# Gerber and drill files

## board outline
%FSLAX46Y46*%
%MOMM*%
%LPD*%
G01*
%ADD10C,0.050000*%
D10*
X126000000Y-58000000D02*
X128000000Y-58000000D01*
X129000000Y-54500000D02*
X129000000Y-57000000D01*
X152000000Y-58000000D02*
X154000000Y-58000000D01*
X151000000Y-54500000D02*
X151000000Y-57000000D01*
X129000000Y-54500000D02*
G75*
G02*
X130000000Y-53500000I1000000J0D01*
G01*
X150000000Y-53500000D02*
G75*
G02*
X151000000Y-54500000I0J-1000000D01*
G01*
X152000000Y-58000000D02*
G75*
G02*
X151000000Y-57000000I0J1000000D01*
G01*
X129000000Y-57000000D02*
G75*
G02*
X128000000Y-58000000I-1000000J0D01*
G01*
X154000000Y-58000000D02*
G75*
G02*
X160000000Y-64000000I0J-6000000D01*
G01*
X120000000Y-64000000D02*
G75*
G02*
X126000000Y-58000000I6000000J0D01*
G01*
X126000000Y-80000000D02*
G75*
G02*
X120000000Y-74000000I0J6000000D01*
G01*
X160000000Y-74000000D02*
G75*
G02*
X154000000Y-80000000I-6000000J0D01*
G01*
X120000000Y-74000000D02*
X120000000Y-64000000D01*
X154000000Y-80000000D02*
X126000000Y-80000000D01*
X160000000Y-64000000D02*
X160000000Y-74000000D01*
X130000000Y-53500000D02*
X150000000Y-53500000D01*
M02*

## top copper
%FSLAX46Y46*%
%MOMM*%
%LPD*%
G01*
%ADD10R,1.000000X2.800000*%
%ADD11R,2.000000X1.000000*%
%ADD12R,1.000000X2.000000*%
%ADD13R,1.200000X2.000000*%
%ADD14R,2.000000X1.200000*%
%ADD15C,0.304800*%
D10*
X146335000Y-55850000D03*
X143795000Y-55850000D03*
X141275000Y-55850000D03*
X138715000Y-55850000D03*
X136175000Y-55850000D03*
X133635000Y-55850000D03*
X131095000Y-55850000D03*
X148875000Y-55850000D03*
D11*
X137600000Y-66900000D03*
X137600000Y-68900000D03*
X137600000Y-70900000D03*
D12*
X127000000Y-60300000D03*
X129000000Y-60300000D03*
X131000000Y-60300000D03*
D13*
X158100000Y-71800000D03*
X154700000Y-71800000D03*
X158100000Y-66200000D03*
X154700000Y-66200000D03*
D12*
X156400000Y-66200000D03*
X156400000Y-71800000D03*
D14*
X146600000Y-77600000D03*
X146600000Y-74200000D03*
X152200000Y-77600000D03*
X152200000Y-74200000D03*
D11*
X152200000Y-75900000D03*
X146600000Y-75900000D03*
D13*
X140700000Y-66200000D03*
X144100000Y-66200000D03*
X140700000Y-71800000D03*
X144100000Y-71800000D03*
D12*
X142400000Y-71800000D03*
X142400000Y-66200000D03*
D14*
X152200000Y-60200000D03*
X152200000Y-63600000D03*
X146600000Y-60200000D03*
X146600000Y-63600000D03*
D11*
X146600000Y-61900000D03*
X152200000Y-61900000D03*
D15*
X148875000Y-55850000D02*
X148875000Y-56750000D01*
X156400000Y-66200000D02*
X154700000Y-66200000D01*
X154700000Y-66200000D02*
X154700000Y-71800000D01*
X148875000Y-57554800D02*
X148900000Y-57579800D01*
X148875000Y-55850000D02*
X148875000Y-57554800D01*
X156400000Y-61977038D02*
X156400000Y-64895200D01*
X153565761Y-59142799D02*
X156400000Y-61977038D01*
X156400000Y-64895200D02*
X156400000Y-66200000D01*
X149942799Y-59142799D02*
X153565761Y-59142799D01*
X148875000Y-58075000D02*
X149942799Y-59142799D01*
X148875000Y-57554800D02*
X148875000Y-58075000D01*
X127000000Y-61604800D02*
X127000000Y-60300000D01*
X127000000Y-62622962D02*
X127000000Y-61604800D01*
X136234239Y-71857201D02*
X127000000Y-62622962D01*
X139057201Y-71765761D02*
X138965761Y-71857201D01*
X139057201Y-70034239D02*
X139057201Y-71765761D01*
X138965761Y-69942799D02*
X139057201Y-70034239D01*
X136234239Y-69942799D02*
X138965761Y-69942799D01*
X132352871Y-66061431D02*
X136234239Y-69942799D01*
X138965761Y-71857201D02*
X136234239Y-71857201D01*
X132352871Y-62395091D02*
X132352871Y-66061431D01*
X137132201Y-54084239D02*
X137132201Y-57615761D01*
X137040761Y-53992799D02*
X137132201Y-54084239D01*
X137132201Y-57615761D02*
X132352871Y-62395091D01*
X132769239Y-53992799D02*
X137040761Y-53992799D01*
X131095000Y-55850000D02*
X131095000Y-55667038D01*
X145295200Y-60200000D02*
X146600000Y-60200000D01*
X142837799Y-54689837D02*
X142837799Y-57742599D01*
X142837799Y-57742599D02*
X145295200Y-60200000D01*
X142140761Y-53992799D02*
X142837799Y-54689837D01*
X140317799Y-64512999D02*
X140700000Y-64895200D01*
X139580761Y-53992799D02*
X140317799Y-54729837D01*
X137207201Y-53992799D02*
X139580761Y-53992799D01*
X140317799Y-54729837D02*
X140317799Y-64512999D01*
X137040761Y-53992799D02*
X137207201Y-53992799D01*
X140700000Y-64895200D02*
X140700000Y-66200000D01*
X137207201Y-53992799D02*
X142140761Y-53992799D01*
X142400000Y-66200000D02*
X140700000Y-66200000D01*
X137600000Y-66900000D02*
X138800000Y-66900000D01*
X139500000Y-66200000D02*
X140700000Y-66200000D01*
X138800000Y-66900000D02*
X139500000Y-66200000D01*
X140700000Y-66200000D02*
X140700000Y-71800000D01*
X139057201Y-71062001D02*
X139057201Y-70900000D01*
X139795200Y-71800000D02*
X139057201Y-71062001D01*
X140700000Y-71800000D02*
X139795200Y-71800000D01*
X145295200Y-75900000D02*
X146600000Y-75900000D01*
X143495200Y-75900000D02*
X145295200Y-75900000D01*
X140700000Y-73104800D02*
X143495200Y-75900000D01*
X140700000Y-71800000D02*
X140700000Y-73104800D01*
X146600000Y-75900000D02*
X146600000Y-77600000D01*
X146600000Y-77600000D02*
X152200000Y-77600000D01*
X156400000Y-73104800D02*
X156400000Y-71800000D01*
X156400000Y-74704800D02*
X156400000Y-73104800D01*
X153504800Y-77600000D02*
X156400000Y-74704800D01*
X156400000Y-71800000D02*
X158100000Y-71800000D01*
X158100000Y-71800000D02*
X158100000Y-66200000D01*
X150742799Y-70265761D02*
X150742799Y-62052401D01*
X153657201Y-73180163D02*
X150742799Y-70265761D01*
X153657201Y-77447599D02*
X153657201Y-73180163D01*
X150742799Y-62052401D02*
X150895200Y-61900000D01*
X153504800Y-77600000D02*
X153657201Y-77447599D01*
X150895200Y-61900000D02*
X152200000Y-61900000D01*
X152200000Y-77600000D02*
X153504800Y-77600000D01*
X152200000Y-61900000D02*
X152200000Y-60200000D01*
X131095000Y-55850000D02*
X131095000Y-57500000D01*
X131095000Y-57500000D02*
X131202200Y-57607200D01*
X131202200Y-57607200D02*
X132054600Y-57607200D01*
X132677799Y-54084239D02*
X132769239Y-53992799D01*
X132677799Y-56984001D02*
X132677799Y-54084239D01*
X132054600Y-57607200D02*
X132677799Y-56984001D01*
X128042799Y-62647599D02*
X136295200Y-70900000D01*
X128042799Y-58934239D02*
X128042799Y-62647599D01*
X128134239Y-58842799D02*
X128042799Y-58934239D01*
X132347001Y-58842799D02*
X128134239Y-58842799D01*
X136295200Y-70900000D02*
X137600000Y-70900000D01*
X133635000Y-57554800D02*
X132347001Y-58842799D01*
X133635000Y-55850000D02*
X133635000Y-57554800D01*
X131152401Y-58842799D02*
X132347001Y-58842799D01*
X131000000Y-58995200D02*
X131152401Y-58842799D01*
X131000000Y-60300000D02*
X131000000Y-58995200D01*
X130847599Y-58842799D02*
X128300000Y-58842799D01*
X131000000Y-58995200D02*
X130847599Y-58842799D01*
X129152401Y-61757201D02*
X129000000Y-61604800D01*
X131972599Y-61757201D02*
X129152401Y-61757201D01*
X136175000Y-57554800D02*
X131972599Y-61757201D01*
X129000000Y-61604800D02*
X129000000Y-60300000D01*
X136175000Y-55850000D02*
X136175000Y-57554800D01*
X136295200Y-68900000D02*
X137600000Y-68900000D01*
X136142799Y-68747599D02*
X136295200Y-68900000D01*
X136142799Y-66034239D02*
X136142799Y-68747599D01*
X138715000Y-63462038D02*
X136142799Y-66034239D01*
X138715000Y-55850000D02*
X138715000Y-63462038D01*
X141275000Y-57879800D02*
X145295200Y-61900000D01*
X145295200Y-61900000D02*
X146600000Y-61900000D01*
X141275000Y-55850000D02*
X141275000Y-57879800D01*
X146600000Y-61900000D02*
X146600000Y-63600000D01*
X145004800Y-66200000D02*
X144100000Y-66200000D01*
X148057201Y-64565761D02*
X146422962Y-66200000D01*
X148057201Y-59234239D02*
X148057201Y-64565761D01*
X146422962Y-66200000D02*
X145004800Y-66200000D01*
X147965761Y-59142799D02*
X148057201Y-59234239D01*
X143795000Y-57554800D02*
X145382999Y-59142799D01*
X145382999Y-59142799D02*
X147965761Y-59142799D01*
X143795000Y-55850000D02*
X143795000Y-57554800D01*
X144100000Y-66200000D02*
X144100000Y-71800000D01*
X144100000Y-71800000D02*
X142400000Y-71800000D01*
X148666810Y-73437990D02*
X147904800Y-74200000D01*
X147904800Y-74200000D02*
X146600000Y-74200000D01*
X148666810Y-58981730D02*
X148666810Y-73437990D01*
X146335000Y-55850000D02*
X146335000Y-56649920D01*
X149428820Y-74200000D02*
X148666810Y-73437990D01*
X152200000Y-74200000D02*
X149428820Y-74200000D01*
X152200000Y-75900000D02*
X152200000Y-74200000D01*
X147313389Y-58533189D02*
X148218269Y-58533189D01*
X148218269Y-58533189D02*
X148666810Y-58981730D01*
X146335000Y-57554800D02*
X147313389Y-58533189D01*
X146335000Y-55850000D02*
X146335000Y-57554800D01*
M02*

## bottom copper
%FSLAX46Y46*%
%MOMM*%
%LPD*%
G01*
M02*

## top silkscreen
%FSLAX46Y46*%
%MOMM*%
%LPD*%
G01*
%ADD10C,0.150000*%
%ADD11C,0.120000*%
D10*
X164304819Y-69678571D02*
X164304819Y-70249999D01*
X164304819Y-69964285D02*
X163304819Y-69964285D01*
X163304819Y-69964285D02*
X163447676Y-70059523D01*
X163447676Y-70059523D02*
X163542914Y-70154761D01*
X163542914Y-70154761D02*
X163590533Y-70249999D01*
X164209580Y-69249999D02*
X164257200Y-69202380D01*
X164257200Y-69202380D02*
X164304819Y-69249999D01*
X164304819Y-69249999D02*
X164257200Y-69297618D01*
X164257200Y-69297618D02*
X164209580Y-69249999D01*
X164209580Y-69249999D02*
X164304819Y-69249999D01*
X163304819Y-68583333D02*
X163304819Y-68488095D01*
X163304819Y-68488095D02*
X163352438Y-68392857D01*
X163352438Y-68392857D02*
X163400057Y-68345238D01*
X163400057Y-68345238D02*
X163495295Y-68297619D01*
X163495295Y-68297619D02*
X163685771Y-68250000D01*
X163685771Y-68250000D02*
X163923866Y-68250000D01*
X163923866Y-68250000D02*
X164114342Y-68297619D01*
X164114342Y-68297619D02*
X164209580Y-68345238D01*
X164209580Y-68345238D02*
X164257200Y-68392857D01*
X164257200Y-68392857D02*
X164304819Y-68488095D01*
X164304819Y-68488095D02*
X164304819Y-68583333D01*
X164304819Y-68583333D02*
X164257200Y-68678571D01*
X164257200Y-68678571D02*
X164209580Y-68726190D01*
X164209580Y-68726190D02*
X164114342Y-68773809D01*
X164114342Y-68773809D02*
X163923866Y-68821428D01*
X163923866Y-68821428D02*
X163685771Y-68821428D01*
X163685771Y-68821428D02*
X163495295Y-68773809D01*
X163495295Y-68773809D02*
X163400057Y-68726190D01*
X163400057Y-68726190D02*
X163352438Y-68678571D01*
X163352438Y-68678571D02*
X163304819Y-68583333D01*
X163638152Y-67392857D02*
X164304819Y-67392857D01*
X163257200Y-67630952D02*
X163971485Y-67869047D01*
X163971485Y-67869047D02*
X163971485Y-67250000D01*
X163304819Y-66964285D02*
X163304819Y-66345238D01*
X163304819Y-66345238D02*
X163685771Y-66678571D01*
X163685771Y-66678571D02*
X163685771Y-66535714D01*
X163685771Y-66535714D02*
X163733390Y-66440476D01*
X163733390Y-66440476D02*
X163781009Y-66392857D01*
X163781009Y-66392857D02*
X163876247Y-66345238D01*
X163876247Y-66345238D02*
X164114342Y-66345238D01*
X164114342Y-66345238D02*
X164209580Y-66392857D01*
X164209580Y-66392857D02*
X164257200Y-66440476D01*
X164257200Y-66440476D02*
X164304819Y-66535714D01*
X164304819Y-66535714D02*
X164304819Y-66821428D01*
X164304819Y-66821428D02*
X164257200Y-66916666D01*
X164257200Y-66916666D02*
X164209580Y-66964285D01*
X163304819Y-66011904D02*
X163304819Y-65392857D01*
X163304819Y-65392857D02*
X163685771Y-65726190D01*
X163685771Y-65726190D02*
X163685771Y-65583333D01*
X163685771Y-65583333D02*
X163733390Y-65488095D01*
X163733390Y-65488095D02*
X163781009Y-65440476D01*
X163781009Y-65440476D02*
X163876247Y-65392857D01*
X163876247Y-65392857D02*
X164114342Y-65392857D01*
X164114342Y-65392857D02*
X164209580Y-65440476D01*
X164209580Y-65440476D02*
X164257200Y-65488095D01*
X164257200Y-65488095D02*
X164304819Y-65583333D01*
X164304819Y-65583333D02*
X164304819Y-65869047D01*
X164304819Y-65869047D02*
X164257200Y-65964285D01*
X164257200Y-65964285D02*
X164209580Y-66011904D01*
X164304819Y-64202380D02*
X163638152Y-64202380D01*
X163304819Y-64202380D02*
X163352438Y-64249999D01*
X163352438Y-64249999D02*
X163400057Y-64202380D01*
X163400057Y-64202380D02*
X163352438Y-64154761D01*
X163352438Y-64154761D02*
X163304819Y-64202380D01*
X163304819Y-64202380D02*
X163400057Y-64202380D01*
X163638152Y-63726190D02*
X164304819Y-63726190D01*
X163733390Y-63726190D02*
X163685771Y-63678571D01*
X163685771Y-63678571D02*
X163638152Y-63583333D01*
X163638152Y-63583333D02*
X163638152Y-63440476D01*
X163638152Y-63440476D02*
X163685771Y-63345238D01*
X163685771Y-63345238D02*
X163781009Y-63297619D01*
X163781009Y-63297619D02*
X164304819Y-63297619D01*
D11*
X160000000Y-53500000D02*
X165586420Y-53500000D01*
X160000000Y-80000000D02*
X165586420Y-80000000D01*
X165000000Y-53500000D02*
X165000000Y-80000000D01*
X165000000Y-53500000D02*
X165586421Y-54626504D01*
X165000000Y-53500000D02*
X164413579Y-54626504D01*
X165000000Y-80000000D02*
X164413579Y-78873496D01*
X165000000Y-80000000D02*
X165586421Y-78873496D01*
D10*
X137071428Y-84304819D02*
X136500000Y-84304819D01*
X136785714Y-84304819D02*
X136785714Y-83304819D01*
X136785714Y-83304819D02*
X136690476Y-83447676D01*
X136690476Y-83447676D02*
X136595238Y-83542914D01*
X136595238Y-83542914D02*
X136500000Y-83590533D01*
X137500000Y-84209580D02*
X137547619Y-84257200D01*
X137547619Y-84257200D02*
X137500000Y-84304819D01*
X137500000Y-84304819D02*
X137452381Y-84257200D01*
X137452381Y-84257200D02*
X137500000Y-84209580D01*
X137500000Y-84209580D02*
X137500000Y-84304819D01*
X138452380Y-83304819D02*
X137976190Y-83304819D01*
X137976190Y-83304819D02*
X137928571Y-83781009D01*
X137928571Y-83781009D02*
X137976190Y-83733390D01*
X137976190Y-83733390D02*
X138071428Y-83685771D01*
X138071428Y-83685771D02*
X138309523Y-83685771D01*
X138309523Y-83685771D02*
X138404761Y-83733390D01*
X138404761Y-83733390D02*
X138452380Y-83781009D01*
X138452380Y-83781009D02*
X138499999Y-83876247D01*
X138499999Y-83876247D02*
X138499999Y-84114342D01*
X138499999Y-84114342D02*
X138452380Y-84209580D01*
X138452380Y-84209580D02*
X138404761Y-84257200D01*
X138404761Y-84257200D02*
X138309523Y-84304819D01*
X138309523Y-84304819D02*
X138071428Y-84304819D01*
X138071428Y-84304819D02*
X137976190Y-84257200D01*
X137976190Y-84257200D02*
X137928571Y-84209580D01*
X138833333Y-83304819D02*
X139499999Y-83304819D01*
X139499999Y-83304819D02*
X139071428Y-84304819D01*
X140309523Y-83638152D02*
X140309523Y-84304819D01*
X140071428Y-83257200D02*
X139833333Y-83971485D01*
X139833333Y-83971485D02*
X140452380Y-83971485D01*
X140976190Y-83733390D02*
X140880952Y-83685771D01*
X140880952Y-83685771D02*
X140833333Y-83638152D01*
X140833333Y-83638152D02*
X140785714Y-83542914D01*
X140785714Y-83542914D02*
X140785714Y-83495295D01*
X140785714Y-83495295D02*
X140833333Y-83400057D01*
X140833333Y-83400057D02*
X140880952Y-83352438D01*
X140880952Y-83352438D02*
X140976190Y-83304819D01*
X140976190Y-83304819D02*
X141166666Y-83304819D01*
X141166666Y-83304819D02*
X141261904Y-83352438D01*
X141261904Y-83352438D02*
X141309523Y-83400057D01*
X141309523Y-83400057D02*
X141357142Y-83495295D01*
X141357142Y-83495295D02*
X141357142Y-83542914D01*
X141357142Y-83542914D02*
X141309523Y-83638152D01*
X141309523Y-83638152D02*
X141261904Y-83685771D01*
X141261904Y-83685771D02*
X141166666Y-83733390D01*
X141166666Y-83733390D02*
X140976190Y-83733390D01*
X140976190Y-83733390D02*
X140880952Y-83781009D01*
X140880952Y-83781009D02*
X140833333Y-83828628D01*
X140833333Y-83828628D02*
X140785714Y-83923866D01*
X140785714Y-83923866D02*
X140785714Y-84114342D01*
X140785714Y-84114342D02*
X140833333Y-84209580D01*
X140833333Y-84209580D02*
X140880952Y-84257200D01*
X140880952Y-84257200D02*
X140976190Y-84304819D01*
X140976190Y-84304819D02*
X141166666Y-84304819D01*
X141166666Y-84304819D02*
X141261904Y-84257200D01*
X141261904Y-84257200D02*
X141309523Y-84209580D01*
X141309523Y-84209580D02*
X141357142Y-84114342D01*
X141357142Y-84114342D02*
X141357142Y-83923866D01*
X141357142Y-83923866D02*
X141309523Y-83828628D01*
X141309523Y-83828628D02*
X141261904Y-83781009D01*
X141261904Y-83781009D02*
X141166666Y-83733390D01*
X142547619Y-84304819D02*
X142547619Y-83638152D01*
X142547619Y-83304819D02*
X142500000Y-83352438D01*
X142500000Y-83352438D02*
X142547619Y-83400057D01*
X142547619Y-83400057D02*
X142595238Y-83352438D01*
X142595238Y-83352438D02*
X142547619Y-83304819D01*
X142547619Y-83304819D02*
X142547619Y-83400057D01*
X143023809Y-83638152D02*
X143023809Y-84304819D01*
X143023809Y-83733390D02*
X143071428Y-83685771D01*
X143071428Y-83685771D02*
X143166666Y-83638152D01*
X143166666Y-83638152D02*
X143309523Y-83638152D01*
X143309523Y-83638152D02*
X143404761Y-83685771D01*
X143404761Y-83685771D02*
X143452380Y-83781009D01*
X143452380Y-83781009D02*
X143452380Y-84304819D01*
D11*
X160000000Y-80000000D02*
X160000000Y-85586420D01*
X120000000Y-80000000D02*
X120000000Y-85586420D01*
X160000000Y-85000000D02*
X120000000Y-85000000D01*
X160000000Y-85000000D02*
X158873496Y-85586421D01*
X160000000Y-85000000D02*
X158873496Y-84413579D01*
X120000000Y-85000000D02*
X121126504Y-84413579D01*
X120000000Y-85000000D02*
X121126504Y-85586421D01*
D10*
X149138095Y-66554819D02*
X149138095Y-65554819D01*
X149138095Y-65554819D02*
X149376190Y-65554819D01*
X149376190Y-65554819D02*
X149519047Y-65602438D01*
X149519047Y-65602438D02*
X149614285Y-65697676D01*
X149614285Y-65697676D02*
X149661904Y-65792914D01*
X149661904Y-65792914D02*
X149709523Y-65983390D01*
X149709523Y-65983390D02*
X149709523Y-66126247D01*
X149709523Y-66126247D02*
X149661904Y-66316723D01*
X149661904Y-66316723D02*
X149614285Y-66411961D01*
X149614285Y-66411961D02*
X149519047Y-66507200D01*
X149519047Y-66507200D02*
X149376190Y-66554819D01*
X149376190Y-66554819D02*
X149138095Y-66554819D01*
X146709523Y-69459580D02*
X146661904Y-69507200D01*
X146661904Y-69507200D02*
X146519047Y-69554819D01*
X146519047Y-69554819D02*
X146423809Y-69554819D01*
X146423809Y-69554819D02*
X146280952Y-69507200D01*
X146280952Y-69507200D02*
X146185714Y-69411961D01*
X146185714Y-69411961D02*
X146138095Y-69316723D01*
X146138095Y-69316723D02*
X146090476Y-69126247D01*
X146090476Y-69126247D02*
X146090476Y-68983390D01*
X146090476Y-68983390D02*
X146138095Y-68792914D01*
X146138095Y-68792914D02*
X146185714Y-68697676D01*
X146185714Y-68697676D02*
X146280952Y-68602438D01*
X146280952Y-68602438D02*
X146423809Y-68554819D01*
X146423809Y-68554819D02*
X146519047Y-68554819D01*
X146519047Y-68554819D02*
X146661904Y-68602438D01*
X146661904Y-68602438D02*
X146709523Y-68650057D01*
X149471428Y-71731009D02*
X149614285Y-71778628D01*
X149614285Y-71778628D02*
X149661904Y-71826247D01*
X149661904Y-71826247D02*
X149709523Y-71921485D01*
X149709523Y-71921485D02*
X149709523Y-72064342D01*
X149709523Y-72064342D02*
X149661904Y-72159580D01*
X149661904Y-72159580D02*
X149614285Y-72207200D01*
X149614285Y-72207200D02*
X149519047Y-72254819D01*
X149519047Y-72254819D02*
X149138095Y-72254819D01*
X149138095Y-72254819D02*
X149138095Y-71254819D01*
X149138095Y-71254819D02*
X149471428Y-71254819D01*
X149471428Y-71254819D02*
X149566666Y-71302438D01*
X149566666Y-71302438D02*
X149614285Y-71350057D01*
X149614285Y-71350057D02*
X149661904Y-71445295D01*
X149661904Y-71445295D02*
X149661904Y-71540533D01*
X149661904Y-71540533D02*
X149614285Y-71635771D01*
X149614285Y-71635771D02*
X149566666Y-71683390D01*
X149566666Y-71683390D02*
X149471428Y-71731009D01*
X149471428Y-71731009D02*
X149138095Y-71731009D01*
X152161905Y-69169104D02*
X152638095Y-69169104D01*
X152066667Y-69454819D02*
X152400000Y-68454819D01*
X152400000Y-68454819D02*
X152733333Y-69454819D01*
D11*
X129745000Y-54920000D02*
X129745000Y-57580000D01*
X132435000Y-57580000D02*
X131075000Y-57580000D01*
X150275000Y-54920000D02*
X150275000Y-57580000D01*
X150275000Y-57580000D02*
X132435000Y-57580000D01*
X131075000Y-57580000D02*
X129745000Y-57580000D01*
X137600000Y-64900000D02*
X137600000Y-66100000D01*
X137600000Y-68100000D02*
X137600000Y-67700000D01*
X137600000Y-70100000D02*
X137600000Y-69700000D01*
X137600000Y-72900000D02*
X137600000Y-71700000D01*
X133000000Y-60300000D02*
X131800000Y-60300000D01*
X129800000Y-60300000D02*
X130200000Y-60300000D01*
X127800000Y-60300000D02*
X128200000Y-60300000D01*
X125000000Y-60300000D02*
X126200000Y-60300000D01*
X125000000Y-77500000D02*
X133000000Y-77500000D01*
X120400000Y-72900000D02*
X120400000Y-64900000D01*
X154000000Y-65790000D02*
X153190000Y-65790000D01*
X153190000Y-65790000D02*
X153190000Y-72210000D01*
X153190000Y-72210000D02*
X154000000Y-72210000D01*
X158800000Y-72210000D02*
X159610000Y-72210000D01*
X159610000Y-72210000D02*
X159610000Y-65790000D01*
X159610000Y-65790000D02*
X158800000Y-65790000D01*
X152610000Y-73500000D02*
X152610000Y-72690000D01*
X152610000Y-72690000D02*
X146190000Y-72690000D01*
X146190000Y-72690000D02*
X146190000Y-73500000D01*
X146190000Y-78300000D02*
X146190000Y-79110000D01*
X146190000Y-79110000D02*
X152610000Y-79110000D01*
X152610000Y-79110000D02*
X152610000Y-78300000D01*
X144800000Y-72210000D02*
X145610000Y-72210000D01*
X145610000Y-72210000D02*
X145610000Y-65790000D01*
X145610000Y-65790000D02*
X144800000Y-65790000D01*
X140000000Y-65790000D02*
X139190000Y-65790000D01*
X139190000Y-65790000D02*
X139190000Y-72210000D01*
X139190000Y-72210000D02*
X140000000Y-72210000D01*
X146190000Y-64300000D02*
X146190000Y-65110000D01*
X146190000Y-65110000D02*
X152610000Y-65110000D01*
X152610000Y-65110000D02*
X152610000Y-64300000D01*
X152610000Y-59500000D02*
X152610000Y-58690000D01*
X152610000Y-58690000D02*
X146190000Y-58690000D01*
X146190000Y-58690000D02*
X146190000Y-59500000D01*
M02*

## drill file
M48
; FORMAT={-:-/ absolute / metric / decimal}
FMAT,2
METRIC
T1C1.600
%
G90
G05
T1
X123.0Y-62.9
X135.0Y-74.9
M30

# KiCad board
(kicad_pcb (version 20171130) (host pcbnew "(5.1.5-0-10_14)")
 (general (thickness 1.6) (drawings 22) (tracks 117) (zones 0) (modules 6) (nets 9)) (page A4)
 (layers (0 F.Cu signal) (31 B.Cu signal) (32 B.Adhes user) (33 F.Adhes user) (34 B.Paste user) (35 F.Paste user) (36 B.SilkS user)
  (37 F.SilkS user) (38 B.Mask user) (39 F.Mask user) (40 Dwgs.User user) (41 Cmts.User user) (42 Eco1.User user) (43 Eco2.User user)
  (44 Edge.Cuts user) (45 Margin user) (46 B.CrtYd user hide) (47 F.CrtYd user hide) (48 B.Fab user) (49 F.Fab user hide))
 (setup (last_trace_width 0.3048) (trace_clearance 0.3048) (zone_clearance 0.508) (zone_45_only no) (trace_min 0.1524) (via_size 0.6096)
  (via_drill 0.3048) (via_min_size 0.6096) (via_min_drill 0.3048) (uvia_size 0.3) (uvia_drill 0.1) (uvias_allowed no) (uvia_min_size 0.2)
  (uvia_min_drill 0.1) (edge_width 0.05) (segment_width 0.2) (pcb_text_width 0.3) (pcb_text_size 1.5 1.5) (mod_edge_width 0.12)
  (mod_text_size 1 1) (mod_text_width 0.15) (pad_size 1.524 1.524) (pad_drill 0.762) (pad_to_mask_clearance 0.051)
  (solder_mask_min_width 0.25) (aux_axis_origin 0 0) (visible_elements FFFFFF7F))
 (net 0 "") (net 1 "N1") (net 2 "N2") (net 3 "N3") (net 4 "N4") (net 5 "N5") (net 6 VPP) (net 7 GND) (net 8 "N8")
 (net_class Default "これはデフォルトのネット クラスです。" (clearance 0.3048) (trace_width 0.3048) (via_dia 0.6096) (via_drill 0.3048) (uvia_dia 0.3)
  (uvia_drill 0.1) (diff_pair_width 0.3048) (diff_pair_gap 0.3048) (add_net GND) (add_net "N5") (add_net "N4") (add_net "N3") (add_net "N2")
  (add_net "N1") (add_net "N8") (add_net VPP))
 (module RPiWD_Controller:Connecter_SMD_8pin (layer F.Cu) (at 148.875 56.25 270)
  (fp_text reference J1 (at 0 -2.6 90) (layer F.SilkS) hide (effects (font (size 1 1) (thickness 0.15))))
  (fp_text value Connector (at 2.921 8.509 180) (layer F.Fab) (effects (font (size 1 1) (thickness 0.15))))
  (fp_line (start -1.33 19.13) (end 1.33 19.13) (layer F.SilkS) (width 0.12))
  (fp_line (start 1.33 16.44) (end 1.33 17.8) (layer F.SilkS) (width 0.12))
  (fp_line (start -1.33 -1.4) (end 1.33 -1.4) (layer F.SilkS) (width 0.12))
  (fp_line (start 1.33 -1.4) (end 1.33 16.44) (layer F.SilkS) (width 0.12))
  (fp_line (start 1.33 17.8) (end 1.33 19.13) (layer F.SilkS) (width 0.12))
  (pad 7 smd rect (at -0.4 2.54 270) (size 2.8 1) (layers F.Cu F.Paste F.Mask) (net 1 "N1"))
  (pad 6 smd rect (at -0.4 5.08 270) (size 2.8 1) (layers F.Cu F.Paste F.Mask) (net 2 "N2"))
  (pad 5 smd rect (at -0.4 7.6 270) (size 2.8 1) (layers F.Cu F.Paste F.Mask) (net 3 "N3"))
  (pad 4 smd rect (at -0.4 10.16 270) (size 2.8 1) (layers F.Cu F.Paste F.Mask) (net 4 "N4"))
  (pad 3 smd rect (at -0.4 12.7 270) (size 2.8 1) (layers F.Cu F.Paste F.Mask) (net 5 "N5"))
  (pad 2 smd rect (at -0.4 15.24 270) (size 2.8 1) (layers F.Cu F.Paste F.Mask) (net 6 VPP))
  (pad 1 smd rect (at -0.4 17.78 270) (size 2.8 1) (layers F.Cu F.Paste F.Mask) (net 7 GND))
  (pad 8 smd rect (at -0.4 0 270) (size 2.8 1) (layers F.Cu F.Paste F.Mask) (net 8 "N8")))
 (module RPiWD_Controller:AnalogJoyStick (layer F.Cu) (at 129 68.9)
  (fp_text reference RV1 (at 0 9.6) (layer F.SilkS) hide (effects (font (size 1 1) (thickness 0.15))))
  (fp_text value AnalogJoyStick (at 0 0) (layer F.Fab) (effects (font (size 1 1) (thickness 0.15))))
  (fp_line (start 8.6 -4) (end 8.6 -2.8) (layer F.SilkS) (width 0.12))
  (fp_line (start 8.6 -0.8) (end 8.6 -1.2) (layer F.SilkS) (width 0.12))
  (fp_line (start 8.6 1.2) (end 8.6 0.8) (layer F.SilkS) (width 0.12))
  (fp_line (start 8.6 4) (end 8.6 2.8) (layer F.SilkS) (width 0.12))
  (fp_line (start 4 -8.6) (end 2.8 -8.6) (layer F.SilkS) (width 0.12))
  (fp_line (start 0.8 -8.6) (end 1.2 -8.6) (layer F.SilkS) (width 0.12))
  (fp_line (start -1.2 -8.6) (end -0.8 -8.6) (layer F.SilkS) (width 0.12))
  (fp_line (start -4 -8.6) (end -2.8 -8.6) (layer F.SilkS) (width 0.12))
  (fp_line (start -4 8.6) (end 4 8.6) (layer F.SilkS) (width 0.12))
  (fp_line (start -8.6 4) (end -8.6 -4) (layer F.SilkS) (width 0.12))
  (pad "" np_thru_hole circle (at 6 6) (size 1.6 1.6) (drill 1.6) (layers *.Cu *.Mask))
  (pad "" np_thru_hole circle (at -6 -6) (size 1.6 1.6) (drill 1.6) (layers *.Cu *.Mask))
  (pad 6 smd rect (at 8.6 -2) (size 2 1) (layers F.Cu F.Paste F.Mask) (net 7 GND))
  (pad 5 smd rect (at 8.6 0) (size 2 1) (layers F.Cu F.Paste F.Mask) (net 4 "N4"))
  (pad 4 smd rect (at 8.6 2) (size 2 1) (layers F.Cu F.Paste F.Mask) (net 6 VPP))
  (pad 3 smd rect (at -2 -8.6) (size 1 2) (layers F.Cu F.Paste F.Mask) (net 7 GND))
  (pad 2 smd rect (at 0 -8.6) (size 1 2) (layers F.Cu F.Paste F.Mask) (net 5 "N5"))
  (pad 1 smd rect (at 2 -8.6) (size 1 2) (layers F.Cu F.Paste F.Mask) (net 6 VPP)))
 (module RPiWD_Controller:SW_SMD (layer F.Cu) (at 156.4 69 270)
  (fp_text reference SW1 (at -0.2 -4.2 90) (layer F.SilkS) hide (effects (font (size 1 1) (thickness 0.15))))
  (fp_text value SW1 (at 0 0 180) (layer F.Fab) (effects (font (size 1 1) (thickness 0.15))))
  (fp_line (start -3.21 2.4) (end -3.21 3.21) (layer F.SilkS) (width 0.12))
  (fp_line (start -3.21 3.21) (end 3.21 3.21) (layer F.SilkS) (width 0.12))
  (fp_line (start 3.21 3.21) (end 3.21 2.4) (layer F.SilkS) (width 0.12))
  (fp_line (start 3.21 -2.4) (end 3.21 -3.21) (layer F.SilkS) (width 0.12))
  (fp_line (start 3.21 -3.21) (end -3.21 -3.21) (layer F.SilkS) (width 0.12))
  (fp_line (start -3.21 -3.21) (end -3.21 -2.4) (layer F.SilkS) (width 0.12))
  (pad 2 smd rect (at 2.8 -1.7 270) (size 2 1.2) (layers F.Cu F.Paste F.Mask) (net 7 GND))
  (pad 1 smd rect (at 2.8 1.7 270) (size 2 1.2) (layers F.Cu F.Paste F.Mask) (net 8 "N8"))
  (pad 2 smd rect (at -2.8 -1.7 270) (size 2 1.2) (layers F.Cu F.Paste F.Mask) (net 7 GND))
  (pad 1 smd rect (at -2.8 1.7 270) (size 2 1.2) (layers F.Cu F.Paste F.Mask) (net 8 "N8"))
  (pad 1 smd rect (at -2.8 0 270) (size 2 1) (layers F.Cu F.Paste F.Mask) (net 8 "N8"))
  (pad 2 smd rect (at 2.8 0 270) (size 2 1) (layers F.Cu F.Paste F.Mask) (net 7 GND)))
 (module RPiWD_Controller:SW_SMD (layer F.Cu) (at 149.4 75.9 180)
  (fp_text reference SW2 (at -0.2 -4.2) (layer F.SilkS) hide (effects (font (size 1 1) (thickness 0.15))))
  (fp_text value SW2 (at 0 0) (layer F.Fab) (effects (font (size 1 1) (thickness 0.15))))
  (fp_line (start -3.21 2.4) (end -3.21 3.21) (layer F.SilkS) (width 0.12))
  (fp_line (start -3.21 3.21) (end 3.21 3.21) (layer F.SilkS) (width 0.12))
  (fp_line (start 3.21 3.21) (end 3.21 2.4) (layer F.SilkS) (width 0.12))
  (fp_line (start 3.21 -2.4) (end 3.21 -3.21) (layer F.SilkS) (width 0.12))
  (fp_line (start 3.21 -3.21) (end -3.21 -3.21) (layer F.SilkS) (width 0.12))
  (fp_line (start -3.21 -3.21) (end -3.21 -2.4) (layer F.SilkS) (width 0.12))
  (pad 2 smd rect (at 2.8 -1.7 180) (size 2 1.2) (layers F.Cu F.Paste F.Mask) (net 7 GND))
  (pad 1 smd rect (at 2.8 1.7 180) (size 2 1.2) (layers F.Cu F.Paste F.Mask) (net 1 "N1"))
  (pad 2 smd rect (at -2.8 -1.7 180) (size 2 1.2) (layers F.Cu F.Paste F.Mask) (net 7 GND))
  (pad 1 smd rect (at -2.8 1.7 180) (size 2 1.2) (layers F.Cu F.Paste F.Mask) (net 1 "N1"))
  (pad 1 smd rect (at -2.8 0 180) (size 2 1) (layers F.Cu F.Paste F.Mask) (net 1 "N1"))
  (pad 2 smd rect (at 2.8 0 180) (size 2 1) (layers F.Cu F.Paste F.Mask) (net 7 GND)))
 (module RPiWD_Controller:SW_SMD (layer F.Cu) (at 142.4 69 90)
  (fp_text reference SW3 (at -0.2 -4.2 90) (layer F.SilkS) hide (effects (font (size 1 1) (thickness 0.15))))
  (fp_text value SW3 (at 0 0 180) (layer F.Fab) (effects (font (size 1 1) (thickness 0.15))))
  (fp_line (start -3.21 2.4) (end -3.21 3.21) (layer F.SilkS) (width 0.12))
  (fp_line (start -3.21 3.21) (end 3.21 3.21) (layer F.SilkS) (width 0.12))
  (fp_line (start 3.21 3.21) (end 3.21 2.4) (layer F.SilkS) (width 0.12))
  (fp_line (start 3.21 -2.4) (end 3.21 -3.21) (layer F.SilkS) (width 0.12))
  (fp_line (start 3.21 -3.21) (end -3.21 -3.21) (layer F.SilkS) (width 0.12))
  (fp_line (start -3.21 -3.21) (end -3.21 -2.4) (layer F.SilkS) (width 0.12))
  (pad 2 smd rect (at 2.8 -1.7 90) (size 2 1.2) (layers F.Cu F.Paste F.Mask) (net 7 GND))
  (pad 1 smd rect (at 2.8 1.7 90) (size 2 1.2) (layers F.Cu F.Paste F.Mask) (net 2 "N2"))
  (pad 2 smd rect (at -2.8 -1.7 90) (size 2 1.2) (layers F.Cu F.Paste F.Mask) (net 7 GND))
  (pad 1 smd rect (at -2.8 1.7 90) (size 2 1.2) (layers F.Cu F.Paste F.Mask) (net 2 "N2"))
  (pad 1 smd rect (at -2.8 0 90) (size 2 1) (layers F.Cu F.Paste F.Mask) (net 2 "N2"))
  (pad 2 smd rect (at 2.8 0 90) (size 2 1) (layers F.Cu F.Paste F.Mask) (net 7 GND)))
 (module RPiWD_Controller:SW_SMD (layer F.Cu) (at 149.4 61.9)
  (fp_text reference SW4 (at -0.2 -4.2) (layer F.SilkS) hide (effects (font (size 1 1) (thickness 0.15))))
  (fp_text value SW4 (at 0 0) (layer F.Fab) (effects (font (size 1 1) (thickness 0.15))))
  (fp_line (start -3.21 2.4) (end -3.21 3.21) (layer F.SilkS) (width 0.12))
  (fp_line (start -3.21 3.21) (end 3.21 3.21) (layer F.SilkS) (width 0.12))
  (fp_line (start 3.21 3.21) (end 3.21 2.4) (layer F.SilkS) (width 0.12))
  (fp_line (start 3.21 -2.4) (end 3.21 -3.21) (layer F.SilkS) (width 0.12))
  (fp_line (start 3.21 -3.21) (end -3.21 -3.21) (layer F.SilkS) (width 0.12))
  (fp_line (start -3.21 -3.21) (end -3.21 -2.4) (layer F.SilkS) (width 0.12))
  (pad 2 smd rect (at 2.8 -1.7) (size 2 1.2) (layers F.Cu F.Paste F.Mask) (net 7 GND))
  (pad 1 smd rect (at 2.8 1.7) (size 2 1.2) (layers F.Cu F.Paste F.Mask) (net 3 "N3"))
  (pad 2 smd rect (at -2.8 -1.7) (size 2 1.2) (layers F.Cu F.Paste F.Mask) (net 7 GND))
  (pad 1 smd rect (at -2.8 1.7) (size 2 1.2) (layers F.Cu F.Paste F.Mask) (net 3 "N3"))
  (pad 1 smd rect (at -2.8 0) (size 2 1) (layers F.Cu F.Paste F.Mask) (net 3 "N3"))
  (pad 2 smd rect (at 2.8 0) (size 2 1) (layers F.Cu F.Paste F.Mask) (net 7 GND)))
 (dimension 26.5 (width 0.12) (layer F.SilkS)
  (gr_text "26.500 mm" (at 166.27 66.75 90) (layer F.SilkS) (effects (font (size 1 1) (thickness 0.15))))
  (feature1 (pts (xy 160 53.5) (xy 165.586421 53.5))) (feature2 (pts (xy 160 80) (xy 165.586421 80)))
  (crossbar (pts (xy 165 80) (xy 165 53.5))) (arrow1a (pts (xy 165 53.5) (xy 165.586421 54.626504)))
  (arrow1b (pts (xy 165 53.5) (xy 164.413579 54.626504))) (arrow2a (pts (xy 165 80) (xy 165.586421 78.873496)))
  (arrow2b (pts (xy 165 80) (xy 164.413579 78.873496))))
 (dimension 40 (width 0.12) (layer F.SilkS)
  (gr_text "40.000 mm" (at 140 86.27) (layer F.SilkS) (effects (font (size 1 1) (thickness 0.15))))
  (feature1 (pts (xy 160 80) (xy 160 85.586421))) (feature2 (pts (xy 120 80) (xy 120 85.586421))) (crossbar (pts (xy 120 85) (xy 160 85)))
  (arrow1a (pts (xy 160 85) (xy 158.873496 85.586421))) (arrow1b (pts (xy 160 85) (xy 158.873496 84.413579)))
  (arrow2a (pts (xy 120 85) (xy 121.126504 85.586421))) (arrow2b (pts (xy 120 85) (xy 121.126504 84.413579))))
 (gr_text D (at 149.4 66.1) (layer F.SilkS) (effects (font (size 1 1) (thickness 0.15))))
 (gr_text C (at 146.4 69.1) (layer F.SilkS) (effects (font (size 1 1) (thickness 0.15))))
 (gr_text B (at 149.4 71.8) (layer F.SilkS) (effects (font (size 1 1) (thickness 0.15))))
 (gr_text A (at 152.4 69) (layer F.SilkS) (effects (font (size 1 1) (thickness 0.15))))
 (gr_line (start 126 58) (end 128 58) (layer Edge.Cuts) (width 0.05))
 (gr_line (start 129 54.5) (end 129 57) (layer Edge.Cuts) (width 0.05))
 (gr_line (start 152 58) (end 154 58) (layer Edge.Cuts) (width 0.05))
 (gr_line (start 151 54.5) (end 151 57) (layer Edge.Cuts) (width 0.05))
 (gr_arc (start 130 54.5) (end 130 53.5) (angle -90) (layer Edge.Cuts) (width 0.05))
 (gr_arc (start 150 54.5) (end 151 54.5) (angle -90) (layer Edge.Cuts) (width 0.05))
 (gr_arc (start 152 57) (end 151 57) (angle -90) (layer Edge.Cuts) (width 0.05))
 (gr_arc (start 128 57) (end 128 58) (angle -90) (layer Edge.Cuts) (width 0.05))
 (gr_arc (start 154 64) (end 160 64) (angle -90) (layer Edge.Cuts) (width 0.05))
 (gr_arc (start 126 64) (end 126 58) (angle -90) (layer Edge.Cuts) (width 0.05))
 (gr_arc (start 126 74) (end 120 74) (angle -90) (layer Edge.Cuts) (width 0.05))
 (gr_arc (start 154 74) (end 154 80) (angle -90) (layer Edge.Cuts) (width 0.05))
 (gr_line (start 120 74) (end 120 64) (layer Edge.Cuts) (width 0.05))
 (gr_line (start 154 80) (end 126 80) (layer Edge.Cuts) (width 0.05))
 (gr_line (start 160 64) (end 160 74) (layer Edge.Cuts) (width 0.05))
 (gr_line (start 130 53.5) (end 150 53.5) (layer Edge.Cuts) (width 0.05))
 (segment (start 148.875 55.85) (end 148.875 56.75) (width 0.3048) (layer F.Cu) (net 8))
 (segment (start 156.4 66.2) (end 154.7 66.2) (width 0.3048) (layer F.Cu) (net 8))
 (segment (start 154.7 66.2) (end 154.7 71.8) (width 0.3048) (layer F.Cu) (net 8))
 (segment (start 148.875 57.5548) (end 148.9 57.5798) (width 0.3048) (layer F.Cu) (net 8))
 (segment (start 148.875 55.85) (end 148.875 57.5548) (width 0.3048) (layer F.Cu) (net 8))
 (segment (start 156.4 61.977038) (end 156.4 64.8952) (width 0.3048) (layer F.Cu) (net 8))
 (segment (start 153.565761 59.142799) (end 156.4 61.977038) (width 0.3048) (layer F.Cu) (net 8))
 (segment (start 156.4 64.8952) (end 156.4 66.2) (width 0.3048) (layer F.Cu) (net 8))
 (segment (start 149.942799 59.142799) (end 153.565761 59.142799) (width 0.3048) (layer F.Cu) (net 8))
 (segment (start 148.875 58.075) (end 149.942799 59.142799) (width 0.3048) (layer F.Cu) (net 8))
 (segment (start 148.875 57.5548) (end 148.875 58.075) (width 0.3048) (layer F.Cu) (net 8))
 (segment (start 127 61.6048) (end 127 60.3) (width 0.3048) (layer F.Cu) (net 7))
 (segment (start 127 62.622962) (end 127 61.6048) (width 0.3048) (layer F.Cu) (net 7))
 (segment (start 136.234239 71.857201) (end 127 62.622962) (width 0.3048) (layer F.Cu) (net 7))
 (segment (start 139.057201 71.765761) (end 138.965761 71.857201) (width 0.3048) (layer F.Cu) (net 7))
 (segment (start 139.057201 70.034239) (end 139.057201 71.765761) (width 0.3048) (layer F.Cu) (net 7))
 (segment (start 138.965761 69.942799) (end 139.057201 70.034239) (width 0.3048) (layer F.Cu) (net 7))
 (segment (start 136.234239 69.942799) (end 138.965761 69.942799) (width 0.3048) (layer F.Cu) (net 7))
 (segment (start 132.352871 66.061431) (end 136.234239 69.942799) (width 0.3048) (layer F.Cu) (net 7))
 (segment (start 138.965761 71.857201) (end 136.234239 71.857201) (width 0.3048) (layer F.Cu) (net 7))
 (segment (start 132.352871 62.395091) (end 132.352871 66.061431) (width 0.3048) (layer F.Cu) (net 7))
 (segment (start 137.132201 54.084239) (end 137.132201 57.615761) (width 0.3048) (layer F.Cu) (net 7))
 (segment (start 137.040761 53.992799) (end 137.132201 54.084239) (width 0.3048) (layer F.Cu) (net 7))
 (segment (start 137.132201 57.615761) (end 132.352871 62.395091) (width 0.3048) (layer F.Cu) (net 7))
 (segment (start 132.769239 53.992799) (end 137.040761 53.992799) (width 0.3048) (layer F.Cu) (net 7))
 (segment (start 131.095 55.85) (end 131.095 55.667038) (width 0.3048) (layer F.Cu) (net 7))
 (segment (start 145.2952 60.2) (end 146.6 60.2) (width 0.3048) (layer F.Cu) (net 7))
 (segment (start 142.837799 54.689837) (end 142.837799 57.742599) (width 0.3048) (layer F.Cu) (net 7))
 (segment (start 142.837799 57.742599) (end 145.2952 60.2) (width 0.3048) (layer F.Cu) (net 7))
 (segment (start 142.140761 53.992799) (end 142.837799 54.689837) (width 0.3048) (layer F.Cu) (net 7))
 (segment (start 140.317799 64.512999) (end 140.7 64.8952) (width 0.3048) (layer F.Cu) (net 7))
 (segment (start 139.580761 53.992799) (end 140.317799 54.729837) (width 0.3048) (layer F.Cu) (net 7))
 (segment (start 137.207201 53.992799) (end 139.580761 53.992799) (width 0.3048) (layer F.Cu) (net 7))
 (segment (start 140.317799 54.729837) (end 140.317799 64.512999) (width 0.3048) (layer F.Cu) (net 7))
 (segment (start 137.040761 53.992799) (end 137.207201 53.992799) (width 0.3048) (layer F.Cu) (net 7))
 (segment (start 140.7 64.8952) (end 140.7 66.2) (width 0.3048) (layer F.Cu) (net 7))
 (segment (start 137.207201 53.992799) (end 142.140761 53.992799) (width 0.3048) (layer F.Cu) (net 7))
 (segment (start 142.4 66.2) (end 140.7 66.2) (width 0.3048) (layer F.Cu) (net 7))
 (segment (start 137.6 66.9) (end 138.8 66.9) (width 0.3048) (layer F.Cu) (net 7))
 (segment (start 139.5 66.2) (end 140.7 66.2) (width 0.3048) (layer F.Cu) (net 7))
 (segment (start 138.8 66.9) (end 139.5 66.2) (width 0.3048) (layer F.Cu) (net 7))
 (segment (start 140.7 66.2) (end 140.7 71.8) (width 0.3048) (layer F.Cu) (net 7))
 (segment (start 139.057201 71.062001) (end 139.057201 70.9) (width 0.3048) (layer F.Cu) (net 7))
 (segment (start 139.7952 71.8) (end 139.057201 71.062001) (width 0.3048) (layer F.Cu) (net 7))
 (segment (start 140.7 71.8) (end 139.7952 71.8) (width 0.3048) (layer F.Cu) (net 7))
 (segment (start 145.2952 75.9) (end 146.6 75.9) (width 0.3048) (layer F.Cu) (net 7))
 (segment (start 143.4952 75.9) (end 145.2952 75.9) (width 0.3048) (layer F.Cu) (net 7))
 (segment (start 140.7 73.1048) (end 143.4952 75.9) (width 0.3048) (layer F.Cu) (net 7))
 (segment (start 140.7 71.8) (end 140.7 73.1048) (width 0.3048) (layer F.Cu) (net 7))
 (segment (start 146.6 75.9) (end 146.6 77.6) (width 0.3048) (layer F.Cu) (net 7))
 (segment (start 146.6 77.6) (end 152.2 77.6) (width 0.3048) (layer F.Cu) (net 7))
 (segment (start 156.4 73.1048) (end 156.4 71.8) (width 0.3048) (layer F.Cu) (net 7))
 (segment (start 156.4 74.7048) (end 156.4 73.1048) (width 0.3048) (layer F.Cu) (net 7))
 (segment (start 153.5048 77.6) (end 156.4 74.7048) (width 0.3048) (layer F.Cu) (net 7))
 (segment (start 156.4 71.8) (end 158.1 71.8) (width 0.3048) (layer F.Cu) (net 7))
 (segment (start 158.1 71.8) (end 158.1 66.2) (width 0.3048) (layer F.Cu) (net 7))
 (segment (start 150.742799 70.265761) (end 150.742799 62.052401) (width 0.3048) (layer F.Cu) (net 7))
 (segment (start 153.657201 73.180163) (end 150.742799 70.265761) (width 0.3048) (layer F.Cu) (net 7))
 (segment (start 153.657201 77.447599) (end 153.657201 73.180163) (width 0.3048) (layer F.Cu) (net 7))
 (segment (start 150.742799 62.052401) (end 150.8952 61.9) (width 0.3048) (layer F.Cu) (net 7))
 (segment (start 153.5048 77.6) (end 153.657201 77.447599) (width 0.3048) (layer F.Cu) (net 7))
 (segment (start 150.8952 61.9) (end 152.2 61.9) (width 0.3048) (layer F.Cu) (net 7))
 (segment (start 152.2 77.6) (end 153.5048 77.6) (width 0.3048) (layer F.Cu) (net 7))
 (segment (start 152.2 61.9) (end 152.2 60.2) (width 0.3048) (layer F.Cu) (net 7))
 (segment (start 131.095 55.85) (end 131.095 57.5) (width 0.3048) (layer F.Cu) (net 7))
 (segment (start 131.095 57.5) (end 131.2022 57.6072) (width 0.3048) (layer F.Cu) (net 7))
 (segment (start 131.2022 57.6072) (end 132.0546 57.6072) (width 0.3048) (layer F.Cu) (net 7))
 (segment (start 132.677799 54.084239) (end 132.769239 53.992799) (width 0.3048) (layer F.Cu) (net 7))
 (segment (start 132.677799 56.984001) (end 132.677799 54.084239) (width 0.3048) (layer F.Cu) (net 7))
 (segment (start 132.0546 57.6072) (end 132.677799 56.984001) (width 0.3048) (layer F.Cu) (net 7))
 (segment (start 128.042799 62.647599) (end 136.2952 70.9) (width 0.3048) (layer F.Cu) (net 6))
 (segment (start 128.042799 58.934239) (end 128.042799 62.647599) (width 0.3048) (layer F.Cu) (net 6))
 (segment (start 128.134239 58.842799) (end 128.042799 58.934239) (width 0.3048) (layer F.Cu) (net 6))
 (segment (start 132.347001 58.842799) (end 128.134239 58.842799) (width 0.3048) (layer F.Cu) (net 6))
 (segment (start 136.2952 70.9) (end 137.6 70.9) (width 0.3048) (layer F.Cu) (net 6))
 (segment (start 133.635 57.5548) (end 132.347001 58.842799) (width 0.3048) (layer F.Cu) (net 6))
 (segment (start 133.635 55.85) (end 133.635 57.5548) (width 0.3048) (layer F.Cu) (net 6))
 (segment (start 131.152401 58.842799) (end 132.347001 58.842799) (width 0.3048) (layer F.Cu) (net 6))
 (segment (start 131 58.9952) (end 131.152401 58.842799) (width 0.3048) (layer F.Cu) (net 6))
 (segment (start 131 60.3) (end 131 58.9952) (width 0.3048) (layer F.Cu) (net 6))
 (segment (start 130.847599 58.842799) (end 128.3 58.842799) (width 0.3048) (layer F.Cu) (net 6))
 (segment (start 131 58.9952) (end 130.847599 58.842799) (width 0.3048) (layer F.Cu) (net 6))
 (segment (start 129.152401 61.757201) (end 129 61.6048) (width 0.3048) (layer F.Cu) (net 5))
 (segment (start 131.972599 61.757201) (end 129.152401 61.757201) (width 0.3048) (layer F.Cu) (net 5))
 (segment (start 136.175 57.5548) (end 131.972599 61.757201) (width 0.3048) (layer F.Cu) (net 5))
 (segment (start 129 61.6048) (end 129 60.3) (width 0.3048) (layer F.Cu) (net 5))
 (segment (start 136.175 55.85) (end 136.175 57.5548) (width 0.3048) (layer F.Cu) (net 5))
 (segment (start 136.2952 68.9) (end 137.6 68.9) (width 0.3048) (layer F.Cu) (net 4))
 (segment (start 136.142799 68.747599) (end 136.2952 68.9) (width 0.3048) (layer F.Cu) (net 4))
 (segment (start 136.142799 66.034239) (end 136.142799 68.747599) (width 0.3048) (layer F.Cu) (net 4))
 (segment (start 138.715 63.462038) (end 136.142799 66.034239) (width 0.3048) (layer F.Cu) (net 4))
 (segment (start 138.715 55.85) (end 138.715 63.462038) (width 0.3048) (layer F.Cu) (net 4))
 (segment (start 141.275 57.8798) (end 145.2952 61.9) (width 0.3048) (layer F.Cu) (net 3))
 (segment (start 145.2952 61.9) (end 146.6 61.9) (width 0.3048) (layer F.Cu) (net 3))
 (segment (start 141.275 55.85) (end 141.275 57.8798) (width 0.3048) (layer F.Cu) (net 3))
 (segment (start 146.6 61.9) (end 146.6 63.6) (width 0.3048) (layer F.Cu) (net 3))
 (segment (start 145.0048 66.2) (end 144.1 66.2) (width 0.3048) (layer F.Cu) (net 2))
 (segment (start 148.057201 64.565761) (end 146.422962 66.2) (width 0.3048) (layer F.Cu) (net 2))
 (segment (start 148.057201 59.234239) (end 148.057201 64.565761) (width 0.3048) (layer F.Cu) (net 2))
 (segment (start 146.422962 66.2) (end 145.0048 66.2) (width 0.3048) (layer F.Cu) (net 2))
 (segment (start 147.965761 59.142799) (end 148.057201 59.234239) (width 0.3048) (layer F.Cu) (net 2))
 (segment (start 143.795 57.5548) (end 145.382999 59.142799) (width 0.3048) (layer F.Cu) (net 2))
 (segment (start 145.382999 59.142799) (end 147.965761 59.142799) (width 0.3048) (layer F.Cu) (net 2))
 (segment (start 143.795 55.85) (end 143.795 57.5548) (width 0.3048) (layer F.Cu) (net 2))
 (segment (start 144.1 66.2) (end 144.1 71.8) (width 0.3048) (layer F.Cu) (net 2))
 (segment (start 144.1 71.8) (end 142.4 71.8) (width 0.3048) (layer F.Cu) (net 2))
 (segment (start 148.66681 73.43799) (end 147.9048 74.2) (width 0.3048) (layer F.Cu) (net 1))
 (segment (start 147.9048 74.2) (end 146.6 74.2) (width 0.3048) (layer F.Cu) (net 1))
 (segment (start 148.66681 58.98173) (end 148.66681 73.43799) (width 0.3048) (layer F.Cu) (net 1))
 (segment (start 146.335 55.85) (end 146.335 56.64992) (width 0.3048) (layer F.Cu) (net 1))
 (segment (start 149.42882 74.2) (end 148.66681 73.43799) (width 0.3048) (layer F.Cu) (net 1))
 (segment (start 152.2 74.2) (end 149.42882 74.2) (width 0.3048) (layer F.Cu) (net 1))
 (segment (start 152.2 75.9) (end 152.2 74.2) (width 0.3048) (layer F.Cu) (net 1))
 (segment (start 147.313389 58.533189) (end 148.218269 58.533189) (width 0.3048) (layer F.Cu) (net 1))
 (segment (start 148.218269 58.533189) (end 148.66681 58.98173) (width 0.3048) (layer F.Cu) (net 1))
 (segment (start 146.335 57.5548) (end 147.313389 58.533189) (width 0.3048) (layer F.Cu) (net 1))
 (segment (start 146.335 55.85) (end 146.335 57.5548) (width 0.3048) (layer F.Cu) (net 1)))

